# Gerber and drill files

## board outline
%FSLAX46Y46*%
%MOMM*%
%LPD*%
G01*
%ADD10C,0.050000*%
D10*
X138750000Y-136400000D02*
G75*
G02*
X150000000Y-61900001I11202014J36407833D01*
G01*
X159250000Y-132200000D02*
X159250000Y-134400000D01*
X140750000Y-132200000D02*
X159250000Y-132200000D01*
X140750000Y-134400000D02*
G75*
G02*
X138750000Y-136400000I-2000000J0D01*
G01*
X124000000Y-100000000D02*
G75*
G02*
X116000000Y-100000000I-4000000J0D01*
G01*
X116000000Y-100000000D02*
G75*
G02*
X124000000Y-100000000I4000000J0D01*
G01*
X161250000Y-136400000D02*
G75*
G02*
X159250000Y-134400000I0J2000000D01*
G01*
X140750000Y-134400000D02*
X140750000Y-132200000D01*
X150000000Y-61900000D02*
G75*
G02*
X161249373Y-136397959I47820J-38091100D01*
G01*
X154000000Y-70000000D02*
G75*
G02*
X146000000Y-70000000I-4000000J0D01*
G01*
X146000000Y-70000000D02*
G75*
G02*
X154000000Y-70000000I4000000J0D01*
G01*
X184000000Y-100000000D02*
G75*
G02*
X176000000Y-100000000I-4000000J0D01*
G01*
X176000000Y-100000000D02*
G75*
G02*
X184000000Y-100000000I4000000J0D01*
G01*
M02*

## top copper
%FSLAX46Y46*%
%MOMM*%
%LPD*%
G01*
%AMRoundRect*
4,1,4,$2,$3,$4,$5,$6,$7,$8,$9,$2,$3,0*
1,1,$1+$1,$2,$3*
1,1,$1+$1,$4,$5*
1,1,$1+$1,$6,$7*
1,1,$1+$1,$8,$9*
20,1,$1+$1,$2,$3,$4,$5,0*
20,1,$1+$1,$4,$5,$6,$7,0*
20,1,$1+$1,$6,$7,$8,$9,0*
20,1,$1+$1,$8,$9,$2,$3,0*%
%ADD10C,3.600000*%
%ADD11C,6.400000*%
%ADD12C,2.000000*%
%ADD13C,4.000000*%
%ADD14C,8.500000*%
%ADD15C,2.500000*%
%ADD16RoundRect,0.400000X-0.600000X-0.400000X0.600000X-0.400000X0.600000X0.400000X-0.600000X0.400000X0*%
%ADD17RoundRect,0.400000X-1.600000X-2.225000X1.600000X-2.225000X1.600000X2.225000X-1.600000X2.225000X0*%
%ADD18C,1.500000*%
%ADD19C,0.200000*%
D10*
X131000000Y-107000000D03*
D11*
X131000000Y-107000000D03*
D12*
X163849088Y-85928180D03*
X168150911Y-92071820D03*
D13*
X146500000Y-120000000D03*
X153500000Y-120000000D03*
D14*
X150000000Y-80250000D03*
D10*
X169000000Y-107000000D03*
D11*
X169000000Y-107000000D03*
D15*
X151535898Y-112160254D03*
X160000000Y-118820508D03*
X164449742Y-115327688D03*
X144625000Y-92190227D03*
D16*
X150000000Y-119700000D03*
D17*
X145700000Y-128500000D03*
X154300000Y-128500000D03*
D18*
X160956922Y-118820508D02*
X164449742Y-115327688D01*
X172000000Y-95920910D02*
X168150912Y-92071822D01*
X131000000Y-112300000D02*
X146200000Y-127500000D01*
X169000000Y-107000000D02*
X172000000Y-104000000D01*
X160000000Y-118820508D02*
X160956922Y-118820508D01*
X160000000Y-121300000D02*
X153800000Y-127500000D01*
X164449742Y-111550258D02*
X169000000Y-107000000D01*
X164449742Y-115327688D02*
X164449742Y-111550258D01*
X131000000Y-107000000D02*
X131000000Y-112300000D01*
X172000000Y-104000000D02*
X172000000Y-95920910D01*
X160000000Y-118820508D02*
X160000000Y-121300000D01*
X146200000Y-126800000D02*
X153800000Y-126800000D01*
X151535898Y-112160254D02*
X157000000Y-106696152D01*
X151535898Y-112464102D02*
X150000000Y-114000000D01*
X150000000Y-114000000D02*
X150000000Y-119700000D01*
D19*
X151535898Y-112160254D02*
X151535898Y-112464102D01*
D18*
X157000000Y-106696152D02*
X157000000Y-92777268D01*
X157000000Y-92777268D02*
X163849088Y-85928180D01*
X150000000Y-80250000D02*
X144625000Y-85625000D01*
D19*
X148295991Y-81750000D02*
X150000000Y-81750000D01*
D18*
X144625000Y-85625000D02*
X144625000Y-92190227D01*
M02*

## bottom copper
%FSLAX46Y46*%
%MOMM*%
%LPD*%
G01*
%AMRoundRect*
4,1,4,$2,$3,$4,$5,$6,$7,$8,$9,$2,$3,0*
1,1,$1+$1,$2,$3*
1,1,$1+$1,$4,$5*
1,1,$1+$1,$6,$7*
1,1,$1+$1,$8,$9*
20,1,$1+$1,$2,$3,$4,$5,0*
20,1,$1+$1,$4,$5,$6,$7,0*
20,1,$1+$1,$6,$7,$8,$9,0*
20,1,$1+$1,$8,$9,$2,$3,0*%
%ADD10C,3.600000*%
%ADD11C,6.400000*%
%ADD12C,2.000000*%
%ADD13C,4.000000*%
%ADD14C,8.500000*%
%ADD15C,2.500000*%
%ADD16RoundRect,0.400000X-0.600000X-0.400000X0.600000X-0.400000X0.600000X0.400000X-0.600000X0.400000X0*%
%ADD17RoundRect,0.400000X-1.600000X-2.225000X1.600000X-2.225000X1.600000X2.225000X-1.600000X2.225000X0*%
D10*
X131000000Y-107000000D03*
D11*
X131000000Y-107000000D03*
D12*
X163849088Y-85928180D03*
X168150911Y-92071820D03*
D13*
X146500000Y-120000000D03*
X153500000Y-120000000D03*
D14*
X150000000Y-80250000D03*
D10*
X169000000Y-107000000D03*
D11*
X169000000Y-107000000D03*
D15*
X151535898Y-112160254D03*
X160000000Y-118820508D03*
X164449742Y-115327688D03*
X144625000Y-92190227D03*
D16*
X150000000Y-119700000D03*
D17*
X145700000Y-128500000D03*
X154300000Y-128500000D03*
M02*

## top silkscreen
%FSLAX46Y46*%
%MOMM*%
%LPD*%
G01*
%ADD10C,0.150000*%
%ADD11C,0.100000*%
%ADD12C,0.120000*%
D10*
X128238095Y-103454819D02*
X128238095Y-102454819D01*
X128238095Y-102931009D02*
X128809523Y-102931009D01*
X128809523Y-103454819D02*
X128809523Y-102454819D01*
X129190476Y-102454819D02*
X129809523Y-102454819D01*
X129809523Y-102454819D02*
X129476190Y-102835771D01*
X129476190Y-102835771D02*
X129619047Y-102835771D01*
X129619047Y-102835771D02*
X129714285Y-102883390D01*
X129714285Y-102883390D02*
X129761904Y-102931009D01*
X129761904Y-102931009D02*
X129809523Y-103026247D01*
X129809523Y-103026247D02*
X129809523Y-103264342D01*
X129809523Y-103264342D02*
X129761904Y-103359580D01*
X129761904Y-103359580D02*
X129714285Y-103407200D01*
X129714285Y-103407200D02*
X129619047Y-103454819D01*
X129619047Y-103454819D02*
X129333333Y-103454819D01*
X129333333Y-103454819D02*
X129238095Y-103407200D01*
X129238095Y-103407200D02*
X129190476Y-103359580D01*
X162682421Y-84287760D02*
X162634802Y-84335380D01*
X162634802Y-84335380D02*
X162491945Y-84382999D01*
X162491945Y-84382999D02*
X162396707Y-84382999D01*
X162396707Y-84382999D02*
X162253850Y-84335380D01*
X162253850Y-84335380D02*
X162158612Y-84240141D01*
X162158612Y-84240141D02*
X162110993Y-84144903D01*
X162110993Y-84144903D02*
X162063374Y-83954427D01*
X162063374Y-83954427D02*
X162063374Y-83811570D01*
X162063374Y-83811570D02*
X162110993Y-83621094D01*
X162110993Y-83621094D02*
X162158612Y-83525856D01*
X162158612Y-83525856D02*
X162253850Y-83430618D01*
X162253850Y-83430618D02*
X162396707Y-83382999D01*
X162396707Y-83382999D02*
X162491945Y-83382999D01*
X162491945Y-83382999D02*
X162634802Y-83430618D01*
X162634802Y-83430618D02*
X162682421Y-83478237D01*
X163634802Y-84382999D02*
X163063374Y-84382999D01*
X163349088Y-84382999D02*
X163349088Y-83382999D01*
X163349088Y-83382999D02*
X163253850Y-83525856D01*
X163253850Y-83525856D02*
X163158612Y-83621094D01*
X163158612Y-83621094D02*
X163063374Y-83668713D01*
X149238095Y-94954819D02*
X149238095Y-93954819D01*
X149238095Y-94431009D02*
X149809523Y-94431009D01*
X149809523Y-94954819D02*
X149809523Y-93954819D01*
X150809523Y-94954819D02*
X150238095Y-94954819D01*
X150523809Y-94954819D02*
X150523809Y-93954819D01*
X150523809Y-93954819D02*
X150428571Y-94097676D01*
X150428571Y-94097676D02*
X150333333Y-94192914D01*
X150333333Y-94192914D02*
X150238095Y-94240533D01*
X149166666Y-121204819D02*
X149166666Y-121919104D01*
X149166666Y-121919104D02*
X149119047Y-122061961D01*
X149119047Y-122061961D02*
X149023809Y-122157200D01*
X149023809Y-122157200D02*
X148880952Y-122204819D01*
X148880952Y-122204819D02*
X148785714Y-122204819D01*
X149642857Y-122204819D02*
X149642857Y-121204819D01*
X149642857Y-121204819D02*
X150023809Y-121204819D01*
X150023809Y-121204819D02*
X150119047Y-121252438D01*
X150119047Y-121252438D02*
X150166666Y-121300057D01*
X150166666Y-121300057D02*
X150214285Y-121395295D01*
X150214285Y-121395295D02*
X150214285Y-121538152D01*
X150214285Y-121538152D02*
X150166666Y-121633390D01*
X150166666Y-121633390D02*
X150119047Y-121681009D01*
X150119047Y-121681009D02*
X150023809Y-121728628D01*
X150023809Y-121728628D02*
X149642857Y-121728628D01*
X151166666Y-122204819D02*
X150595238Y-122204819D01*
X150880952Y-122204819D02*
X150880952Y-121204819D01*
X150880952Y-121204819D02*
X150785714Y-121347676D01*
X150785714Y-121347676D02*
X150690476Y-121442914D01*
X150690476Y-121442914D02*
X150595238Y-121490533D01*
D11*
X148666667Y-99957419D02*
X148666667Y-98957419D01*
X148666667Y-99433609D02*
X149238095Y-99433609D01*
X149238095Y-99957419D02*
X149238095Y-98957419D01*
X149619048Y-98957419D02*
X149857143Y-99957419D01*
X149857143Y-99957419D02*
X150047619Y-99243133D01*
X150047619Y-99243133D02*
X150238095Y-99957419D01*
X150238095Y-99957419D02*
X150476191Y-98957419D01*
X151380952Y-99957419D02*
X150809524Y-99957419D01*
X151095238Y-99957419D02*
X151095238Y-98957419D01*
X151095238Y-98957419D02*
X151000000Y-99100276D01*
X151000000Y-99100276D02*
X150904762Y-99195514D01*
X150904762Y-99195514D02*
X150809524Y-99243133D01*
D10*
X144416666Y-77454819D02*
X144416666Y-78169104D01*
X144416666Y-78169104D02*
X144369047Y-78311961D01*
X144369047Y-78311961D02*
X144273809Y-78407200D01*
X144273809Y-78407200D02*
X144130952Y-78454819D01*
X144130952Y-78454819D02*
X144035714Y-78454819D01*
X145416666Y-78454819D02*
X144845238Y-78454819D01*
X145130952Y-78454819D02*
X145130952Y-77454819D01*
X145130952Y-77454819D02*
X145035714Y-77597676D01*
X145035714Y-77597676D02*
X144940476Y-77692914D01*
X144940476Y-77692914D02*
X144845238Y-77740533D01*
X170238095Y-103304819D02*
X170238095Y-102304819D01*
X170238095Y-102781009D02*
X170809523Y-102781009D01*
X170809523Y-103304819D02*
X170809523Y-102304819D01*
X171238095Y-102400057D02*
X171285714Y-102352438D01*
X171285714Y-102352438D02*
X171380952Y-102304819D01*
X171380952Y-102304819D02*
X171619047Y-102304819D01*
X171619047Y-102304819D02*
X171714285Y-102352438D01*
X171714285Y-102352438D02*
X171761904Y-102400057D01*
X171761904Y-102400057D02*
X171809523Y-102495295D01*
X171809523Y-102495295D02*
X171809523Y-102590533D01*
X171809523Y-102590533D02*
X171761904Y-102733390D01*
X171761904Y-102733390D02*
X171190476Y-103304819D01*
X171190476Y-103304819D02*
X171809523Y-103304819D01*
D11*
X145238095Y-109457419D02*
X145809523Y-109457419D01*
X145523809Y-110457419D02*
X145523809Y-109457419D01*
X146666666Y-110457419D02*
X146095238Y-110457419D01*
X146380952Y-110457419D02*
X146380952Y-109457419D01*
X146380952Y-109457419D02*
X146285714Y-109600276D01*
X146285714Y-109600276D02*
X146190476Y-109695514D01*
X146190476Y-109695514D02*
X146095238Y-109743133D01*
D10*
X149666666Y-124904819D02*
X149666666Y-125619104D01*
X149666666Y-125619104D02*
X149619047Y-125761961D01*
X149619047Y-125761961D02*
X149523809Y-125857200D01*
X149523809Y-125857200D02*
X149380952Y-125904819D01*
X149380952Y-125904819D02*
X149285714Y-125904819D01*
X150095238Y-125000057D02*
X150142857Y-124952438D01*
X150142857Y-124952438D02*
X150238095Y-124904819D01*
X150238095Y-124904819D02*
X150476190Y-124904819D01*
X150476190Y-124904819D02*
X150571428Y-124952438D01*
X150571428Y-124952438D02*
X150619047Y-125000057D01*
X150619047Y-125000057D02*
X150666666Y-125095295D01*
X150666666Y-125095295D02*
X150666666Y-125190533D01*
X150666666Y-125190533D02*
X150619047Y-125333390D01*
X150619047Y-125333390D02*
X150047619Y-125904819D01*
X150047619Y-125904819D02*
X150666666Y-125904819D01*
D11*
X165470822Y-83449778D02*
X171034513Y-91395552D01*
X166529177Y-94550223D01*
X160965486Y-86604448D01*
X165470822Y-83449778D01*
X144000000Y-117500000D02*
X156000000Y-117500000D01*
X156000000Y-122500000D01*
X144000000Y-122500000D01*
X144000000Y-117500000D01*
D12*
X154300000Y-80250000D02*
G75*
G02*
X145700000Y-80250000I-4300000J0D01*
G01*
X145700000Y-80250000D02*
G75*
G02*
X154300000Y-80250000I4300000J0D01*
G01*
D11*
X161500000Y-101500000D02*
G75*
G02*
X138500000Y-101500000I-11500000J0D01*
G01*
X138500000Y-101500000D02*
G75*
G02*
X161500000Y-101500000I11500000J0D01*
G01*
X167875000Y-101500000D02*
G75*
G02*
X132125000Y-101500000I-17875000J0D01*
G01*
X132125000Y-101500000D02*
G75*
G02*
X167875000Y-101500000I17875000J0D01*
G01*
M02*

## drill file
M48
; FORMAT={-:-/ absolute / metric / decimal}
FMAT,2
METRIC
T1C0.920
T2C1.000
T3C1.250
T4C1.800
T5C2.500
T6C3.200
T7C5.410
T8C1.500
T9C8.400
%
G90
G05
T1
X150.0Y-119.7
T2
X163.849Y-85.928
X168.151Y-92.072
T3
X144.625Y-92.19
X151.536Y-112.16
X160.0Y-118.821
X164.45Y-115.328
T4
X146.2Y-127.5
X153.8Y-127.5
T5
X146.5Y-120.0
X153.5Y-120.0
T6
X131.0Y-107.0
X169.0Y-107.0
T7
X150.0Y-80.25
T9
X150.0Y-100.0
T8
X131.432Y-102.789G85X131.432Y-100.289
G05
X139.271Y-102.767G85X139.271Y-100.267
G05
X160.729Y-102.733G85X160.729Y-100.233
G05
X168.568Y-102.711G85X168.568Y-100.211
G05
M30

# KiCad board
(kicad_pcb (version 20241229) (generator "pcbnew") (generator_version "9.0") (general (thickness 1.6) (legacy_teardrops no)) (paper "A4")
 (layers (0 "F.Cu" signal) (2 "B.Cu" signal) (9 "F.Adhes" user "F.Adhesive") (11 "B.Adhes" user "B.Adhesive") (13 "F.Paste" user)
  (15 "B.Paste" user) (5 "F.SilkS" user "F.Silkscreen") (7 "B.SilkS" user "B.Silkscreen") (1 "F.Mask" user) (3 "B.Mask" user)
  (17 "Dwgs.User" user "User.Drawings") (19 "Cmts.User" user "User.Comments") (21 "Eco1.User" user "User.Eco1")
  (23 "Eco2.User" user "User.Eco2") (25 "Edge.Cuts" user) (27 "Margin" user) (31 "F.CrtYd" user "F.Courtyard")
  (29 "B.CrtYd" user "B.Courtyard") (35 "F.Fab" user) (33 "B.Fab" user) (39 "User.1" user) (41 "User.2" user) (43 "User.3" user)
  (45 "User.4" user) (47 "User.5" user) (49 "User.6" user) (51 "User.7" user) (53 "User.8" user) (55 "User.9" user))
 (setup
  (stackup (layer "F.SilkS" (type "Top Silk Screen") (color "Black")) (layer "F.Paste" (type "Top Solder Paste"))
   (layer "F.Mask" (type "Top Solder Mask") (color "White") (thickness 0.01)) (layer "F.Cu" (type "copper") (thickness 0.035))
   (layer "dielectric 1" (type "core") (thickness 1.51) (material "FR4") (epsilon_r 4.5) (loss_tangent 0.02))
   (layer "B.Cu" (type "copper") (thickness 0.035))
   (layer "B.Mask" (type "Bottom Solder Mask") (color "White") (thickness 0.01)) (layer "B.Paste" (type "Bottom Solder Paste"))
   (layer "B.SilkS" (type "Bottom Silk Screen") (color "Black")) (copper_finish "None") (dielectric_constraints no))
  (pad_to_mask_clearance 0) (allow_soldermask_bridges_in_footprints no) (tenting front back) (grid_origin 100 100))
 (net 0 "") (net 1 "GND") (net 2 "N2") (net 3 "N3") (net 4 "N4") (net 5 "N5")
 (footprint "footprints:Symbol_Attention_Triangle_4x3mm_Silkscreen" (layer "F.Cu") (at 175 111.5)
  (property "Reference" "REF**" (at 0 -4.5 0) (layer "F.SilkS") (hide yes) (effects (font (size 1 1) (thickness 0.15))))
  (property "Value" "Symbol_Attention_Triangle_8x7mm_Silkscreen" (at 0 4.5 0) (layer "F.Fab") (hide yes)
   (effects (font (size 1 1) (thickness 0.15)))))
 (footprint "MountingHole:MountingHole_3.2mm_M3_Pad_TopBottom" (layer "F.Cu") (at 131 107)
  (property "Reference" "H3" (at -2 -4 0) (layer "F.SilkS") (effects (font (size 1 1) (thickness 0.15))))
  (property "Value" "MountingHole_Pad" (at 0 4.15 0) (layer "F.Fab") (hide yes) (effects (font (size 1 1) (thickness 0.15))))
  (pad "1" thru_hole circle (at 0 0) (size 3.6 3.6) (drill 3.2) (layers "*.Cu" "*.Mask") (remove_unused_layers no) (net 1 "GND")
   (zone_connect 2))
  (pad "1" connect circle (at 0 0) (size 6.4 6.4) (layers "F.Cu" "F.Mask") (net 1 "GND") (zone_connect 2))
  (pad "1" connect circle (at 0 0) (size 6.4 6.4) (layers "B.Cu" "B.Mask") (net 1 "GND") (zone_connect 2)))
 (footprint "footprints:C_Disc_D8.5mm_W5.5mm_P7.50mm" (layer "F.Cu") (at 163.849088 85.92818 -55)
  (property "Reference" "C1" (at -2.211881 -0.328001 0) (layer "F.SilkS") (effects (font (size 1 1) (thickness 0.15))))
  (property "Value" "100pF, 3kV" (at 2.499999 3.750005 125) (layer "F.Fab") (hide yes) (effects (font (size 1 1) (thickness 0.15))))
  (fp_poly
   (pts (xy -1.1 -2.75) (xy 8.599999 -2.75) (xy 8.6 2.75) (xy -1.1 2.75)) (stroke (width 0.1) (type solid)) (fill no) (layer "F.SilkS"))
  (pad "1" thru_hole circle (at 0 0 305) (size 2 2) (drill 1) (layers "*.Cu" "*.Mask") (remove_unused_layers no) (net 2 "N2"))
  (pad "2" thru_hole circle (at 7.5 0 305) (size 2 2) (drill 1) (layers "*.Cu" "*.Mask") (remove_unused_layers no) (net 1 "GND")))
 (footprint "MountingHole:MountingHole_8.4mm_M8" (layer "F.Cu") (at 150 100)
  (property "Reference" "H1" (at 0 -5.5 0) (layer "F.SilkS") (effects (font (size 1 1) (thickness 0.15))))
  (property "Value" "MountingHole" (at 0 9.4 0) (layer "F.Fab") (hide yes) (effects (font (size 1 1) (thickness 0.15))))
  (pad "" np_thru_hole circle (at 0 0) (size 8.4 8.4) (drill 8.4) (layers "*.Cu" "*.Mask")))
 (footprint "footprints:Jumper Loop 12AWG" (layer "F.Cu") (at 146.5 120)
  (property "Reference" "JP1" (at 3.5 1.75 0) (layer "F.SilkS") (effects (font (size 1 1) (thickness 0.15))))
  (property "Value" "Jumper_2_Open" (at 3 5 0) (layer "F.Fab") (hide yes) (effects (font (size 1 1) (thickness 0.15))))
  (fp_rect (start -2.5 -2.5) (end 9.5 2.5) (stroke (width 0.1) (type solid)) (fill no) (layer "F.SilkS"))
  (pad "1" thru_hole circle (at 0 0) (size 4 4) (drill 2.5) (layers "*.Cu" "*.Mask") (remove_unused_layers no) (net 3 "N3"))
  (pad "2" thru_hole circle (at 7 0) (size 4 4) (drill 2.5) (layers "*.Cu" "*.Mask") (remove_unused_layers no) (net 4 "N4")))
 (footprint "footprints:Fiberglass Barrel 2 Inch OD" (layer "F.Cu") (at 150 100)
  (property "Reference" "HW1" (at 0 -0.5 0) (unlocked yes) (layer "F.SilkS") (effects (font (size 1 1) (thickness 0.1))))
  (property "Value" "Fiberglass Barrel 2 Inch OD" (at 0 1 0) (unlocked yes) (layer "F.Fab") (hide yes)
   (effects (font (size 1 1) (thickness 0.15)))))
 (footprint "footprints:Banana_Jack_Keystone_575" (layer "F.Cu") (at 150 80.25)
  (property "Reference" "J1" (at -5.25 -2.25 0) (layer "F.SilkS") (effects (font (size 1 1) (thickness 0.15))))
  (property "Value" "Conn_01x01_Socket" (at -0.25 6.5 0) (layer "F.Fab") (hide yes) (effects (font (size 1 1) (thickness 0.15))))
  (fp_circle (center 0 0) (end 4.3 0) (stroke (width 0.12) (type solid)) (fill no) (layer "F.SilkS"))
  (pad "1" thru_hole circle (at 0 0) (size 8.5 8.5) (drill 5.41) (layers "*.Cu" "*.Mask") (remove_unused_layers no) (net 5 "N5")))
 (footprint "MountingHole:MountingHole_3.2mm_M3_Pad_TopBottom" (layer "F.Cu") (at 169 107)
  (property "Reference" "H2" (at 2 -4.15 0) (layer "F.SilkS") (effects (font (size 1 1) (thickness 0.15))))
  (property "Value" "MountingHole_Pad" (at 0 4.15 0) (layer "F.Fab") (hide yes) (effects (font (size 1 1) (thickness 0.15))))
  (pad "1" thru_hole circle (at 0 0) (size 3.6 3.6) (drill 3.2) (layers "*.Cu" "*.Mask") (remove_unused_layers no) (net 1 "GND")
   (zone_connect 2))
  (pad "1" connect circle (at 0 0) (size 6.4 6.4) (layers "F.Cu" "F.Mask") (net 1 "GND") (zone_connect 2))
  (pad "1" connect circle (at 0 0) (size 6.4 6.4) (layers "B.Cu" "B.Mask") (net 1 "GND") (zone_connect 2)))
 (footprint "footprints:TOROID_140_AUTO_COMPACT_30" (layer "F.Cu") (at 150 101.5 30)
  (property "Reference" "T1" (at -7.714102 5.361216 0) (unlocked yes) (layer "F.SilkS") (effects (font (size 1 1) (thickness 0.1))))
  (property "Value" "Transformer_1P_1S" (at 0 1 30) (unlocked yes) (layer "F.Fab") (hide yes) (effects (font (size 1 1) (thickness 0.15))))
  (fp_circle (center 0 0) (end 11.5 0) (stroke (width 0.1) (type default)) (fill no) (layer "F.SilkS"))
  (fp_circle (center 0 0) (end 17.875 0) (stroke (width 0.1) (type default)) (fill no) (layer "F.SilkS"))
  (pad "" np_thru_hole rect (at -16.1 -9.25 90) (size 5 3) (drill oval 4 1.5) (layers))
  (pad "" np_thru_hole rect (at -9.3 -5.35 90) (size 5 3) (drill oval 4 1.5) (layers))
  (pad "" np_thru_hole rect (at 9.3 5.35 90) (size 5 3) (drill oval 4 1.5) (layers))
  (pad "" np_thru_hole rect (at 16.1 9.25 90) (size 5 3) (drill oval 4 1.5) (layers))
  (pad "1" thru_hole circle (at -4 10 30) (size 2.5 2.5) (drill 1.25) (layers "*.Cu" "*.Mask") (remove_unused_layers no) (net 2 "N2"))
  (pad "2" thru_hole circle (at 0 20 30) (size 2.5 2.5) (drill 1.25) (layers "*.Cu" "*.Mask") (remove_unused_layers no) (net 1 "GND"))
  (pad "3" thru_hole circle (at 5.6 19.2 30) (size 2.5 2.5) (drill 1.25) (layers "*.Cu" "*.Mask") (remove_unused_layers no) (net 1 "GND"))
  (pad "4" thru_hole circle (at 0 -10.75 30) (size 2.5 2.5) (drill 1.25) (layers "*.Cu" "*.Mask") (remove_unused_layers no) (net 5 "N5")))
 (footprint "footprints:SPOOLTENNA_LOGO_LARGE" (layer "B.Cu") (at 150 89 180)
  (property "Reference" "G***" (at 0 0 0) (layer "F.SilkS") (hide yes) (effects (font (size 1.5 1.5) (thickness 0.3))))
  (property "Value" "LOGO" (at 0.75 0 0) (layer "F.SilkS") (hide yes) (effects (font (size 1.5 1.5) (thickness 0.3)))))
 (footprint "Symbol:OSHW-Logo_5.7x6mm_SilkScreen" (layer "B.Cu") (at 166 127 180)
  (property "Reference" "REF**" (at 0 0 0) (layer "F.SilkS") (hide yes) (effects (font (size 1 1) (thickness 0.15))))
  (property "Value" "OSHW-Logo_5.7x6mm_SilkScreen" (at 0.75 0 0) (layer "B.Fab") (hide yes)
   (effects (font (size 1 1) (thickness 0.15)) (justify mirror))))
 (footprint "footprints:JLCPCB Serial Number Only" (layer "B.Cu") (at 126 118 180)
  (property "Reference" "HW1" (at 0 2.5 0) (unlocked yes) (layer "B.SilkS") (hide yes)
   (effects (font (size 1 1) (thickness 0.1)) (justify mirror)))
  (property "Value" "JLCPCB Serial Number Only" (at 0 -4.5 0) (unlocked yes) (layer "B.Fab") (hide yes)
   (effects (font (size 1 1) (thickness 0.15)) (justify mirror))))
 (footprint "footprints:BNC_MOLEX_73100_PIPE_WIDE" (layer "B.Cu") (at 150 119.7)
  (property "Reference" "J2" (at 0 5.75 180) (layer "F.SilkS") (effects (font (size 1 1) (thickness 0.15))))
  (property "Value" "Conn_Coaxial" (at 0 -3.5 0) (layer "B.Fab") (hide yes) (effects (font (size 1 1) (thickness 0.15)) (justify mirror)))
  (pad "1" thru_hole roundrect (at 0 0) (size 2 1.6) (drill 0.92) (layers "*.Cu" "*.Mask") (remove_unused_layers no) (roundrect_rratio 0.25)
   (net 2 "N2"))
  (pad "2" thru_hole roundrect (at -3.8 7.8) (size 4 5.25) (drill 1.8 (offset -0.5 1)) (layers "*.Cu" "*.Mask") (remove_unused_layers no)
   (roundrect_rratio 0.1) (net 1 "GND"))
  (pad "2" thru_hole roundrect (at 3.8 7.8) (size 4 5.25) (drill 1.8 (offset 0.5 1)) (layers "*.Cu" "*.Mask") (remove_unused_layers no)
   (roundrect_rratio 0.1) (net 1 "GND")))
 (gr_arc (start 138.75 136.4) (mid 112.286837 94.304471) (end 150 61.9) (stroke (width 0.05) (type default)) (layer "Edge.Cuts"))
 (gr_line (start 159.25 132.2) (end 159.25 134.4) (stroke (width 0.05) (type solid)) (layer "Edge.Cuts"))
 (gr_line (start 140.75 132.2) (end 159.25 132.2) (stroke (width 0.05) (type solid)) (layer "Edge.Cuts"))
 (gr_arc (start 140.75 134.4) (mid 140.164214 135.814214) (end 138.75 136.4) (stroke (width 0.05) (type default)) (layer "Edge.Cuts"))
 (gr_circle (center 120 100) (end 124 100) (stroke (width 0.05) (type default)) (fill no) (layer "Edge.Cuts"))
 (gr_arc (start 161.25 136.4) (mid 159.835785 135.814214) (end 159.25 134.4) (stroke (width 0.05) (type default)) (layer "Edge.Cuts"))
 (gr_line (start 140.75 134.4) (end 140.75 132.2) (stroke (width 0.05) (type solid)) (layer "Edge.Cuts"))
 (gr_arc (start 150 61.9) (mid 187.711966 94.30372) (end 161.249371 136.397954) (stroke (width 0.05) (type default)) (layer "Edge.Cuts"))
 (gr_circle (center 150 70) (end 154 70) (stroke (width 0.05) (type default)) (fill no) (layer "Edge.Cuts"))
 (gr_circle (center 180 100) (end 184 100) (stroke (width 0.05) (type solid)) (fill no) (layer "Edge.Cuts"))
 (segment (start 160.956922 118.820508) (end 164.449742 115.327688) (width 1.5) (layer "F.Cu") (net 1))
 (segment (start 172 95.92091) (end 168.150912 92.071822) (width 1.5) (layer "F.Cu") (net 1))
 (segment (start 131 112.3) (end 146.2 127.5) (width 1.5) (layer "F.Cu") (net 1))
 (segment (start 169 107) (end 172 104) (width 1.5) (layer "F.Cu") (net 1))
 (segment (start 160 118.820508) (end 160.956922 118.820508) (width 1.5) (layer "F.Cu") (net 1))
 (segment (start 160 121.3) (end 153.8 127.5) (width 1.5) (layer "F.Cu") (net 1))
 (segment (start 164.449742 111.550258) (end 169 107) (width 1.5) (layer "F.Cu") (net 1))
 (segment (start 164.449742 115.327688) (end 164.449742 111.550258) (width 1.5) (layer "F.Cu") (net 1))
 (segment (start 131 107) (end 131 112.3) (width 1.5) (layer "F.Cu") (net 1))
 (segment (start 172 104) (end 172 95.92091) (width 1.5) (layer "F.Cu") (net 1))
 (segment (start 160 118.820508) (end 160 121.3) (width 1.5) (layer "F.Cu") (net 1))
 (segment (start 146.2 126.8) (end 153.8 126.8) (width 1.5) (layer "F.Cu") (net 1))
 (segment (start 151.535898 112.160254) (end 157 106.696152) (width 1.5) (layer "F.Cu") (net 2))
 (segment (start 151.535898 112.464102) (end 150 114) (width 1.5) (layer "F.Cu") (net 2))
 (segment (start 150 114) (end 150 119.7) (width 1.5) (layer "F.Cu") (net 2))
 (segment (start 151.535898 112.160254) (end 151.535898 112.464102) (width 0.2) (layer "F.Cu") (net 2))
 (segment (start 157 106.696152) (end 157 92.777268) (width 1.5) (layer "F.Cu") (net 2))
 (segment (start 157 92.777268) (end 163.849088 85.92818) (width 1.5) (layer "F.Cu") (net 2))
 (segment (start 150 80.25) (end 144.625 85.625) (width 1.5) (layer "F.Cu") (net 5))
 (segment (start 148.295991 81.75) (end 150 81.75) (width 0.2) (layer "F.Cu") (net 5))
 (segment (start 144.625 85.625) (end 144.625 92.190227) (width 1.5) (layer "F.Cu") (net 5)))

